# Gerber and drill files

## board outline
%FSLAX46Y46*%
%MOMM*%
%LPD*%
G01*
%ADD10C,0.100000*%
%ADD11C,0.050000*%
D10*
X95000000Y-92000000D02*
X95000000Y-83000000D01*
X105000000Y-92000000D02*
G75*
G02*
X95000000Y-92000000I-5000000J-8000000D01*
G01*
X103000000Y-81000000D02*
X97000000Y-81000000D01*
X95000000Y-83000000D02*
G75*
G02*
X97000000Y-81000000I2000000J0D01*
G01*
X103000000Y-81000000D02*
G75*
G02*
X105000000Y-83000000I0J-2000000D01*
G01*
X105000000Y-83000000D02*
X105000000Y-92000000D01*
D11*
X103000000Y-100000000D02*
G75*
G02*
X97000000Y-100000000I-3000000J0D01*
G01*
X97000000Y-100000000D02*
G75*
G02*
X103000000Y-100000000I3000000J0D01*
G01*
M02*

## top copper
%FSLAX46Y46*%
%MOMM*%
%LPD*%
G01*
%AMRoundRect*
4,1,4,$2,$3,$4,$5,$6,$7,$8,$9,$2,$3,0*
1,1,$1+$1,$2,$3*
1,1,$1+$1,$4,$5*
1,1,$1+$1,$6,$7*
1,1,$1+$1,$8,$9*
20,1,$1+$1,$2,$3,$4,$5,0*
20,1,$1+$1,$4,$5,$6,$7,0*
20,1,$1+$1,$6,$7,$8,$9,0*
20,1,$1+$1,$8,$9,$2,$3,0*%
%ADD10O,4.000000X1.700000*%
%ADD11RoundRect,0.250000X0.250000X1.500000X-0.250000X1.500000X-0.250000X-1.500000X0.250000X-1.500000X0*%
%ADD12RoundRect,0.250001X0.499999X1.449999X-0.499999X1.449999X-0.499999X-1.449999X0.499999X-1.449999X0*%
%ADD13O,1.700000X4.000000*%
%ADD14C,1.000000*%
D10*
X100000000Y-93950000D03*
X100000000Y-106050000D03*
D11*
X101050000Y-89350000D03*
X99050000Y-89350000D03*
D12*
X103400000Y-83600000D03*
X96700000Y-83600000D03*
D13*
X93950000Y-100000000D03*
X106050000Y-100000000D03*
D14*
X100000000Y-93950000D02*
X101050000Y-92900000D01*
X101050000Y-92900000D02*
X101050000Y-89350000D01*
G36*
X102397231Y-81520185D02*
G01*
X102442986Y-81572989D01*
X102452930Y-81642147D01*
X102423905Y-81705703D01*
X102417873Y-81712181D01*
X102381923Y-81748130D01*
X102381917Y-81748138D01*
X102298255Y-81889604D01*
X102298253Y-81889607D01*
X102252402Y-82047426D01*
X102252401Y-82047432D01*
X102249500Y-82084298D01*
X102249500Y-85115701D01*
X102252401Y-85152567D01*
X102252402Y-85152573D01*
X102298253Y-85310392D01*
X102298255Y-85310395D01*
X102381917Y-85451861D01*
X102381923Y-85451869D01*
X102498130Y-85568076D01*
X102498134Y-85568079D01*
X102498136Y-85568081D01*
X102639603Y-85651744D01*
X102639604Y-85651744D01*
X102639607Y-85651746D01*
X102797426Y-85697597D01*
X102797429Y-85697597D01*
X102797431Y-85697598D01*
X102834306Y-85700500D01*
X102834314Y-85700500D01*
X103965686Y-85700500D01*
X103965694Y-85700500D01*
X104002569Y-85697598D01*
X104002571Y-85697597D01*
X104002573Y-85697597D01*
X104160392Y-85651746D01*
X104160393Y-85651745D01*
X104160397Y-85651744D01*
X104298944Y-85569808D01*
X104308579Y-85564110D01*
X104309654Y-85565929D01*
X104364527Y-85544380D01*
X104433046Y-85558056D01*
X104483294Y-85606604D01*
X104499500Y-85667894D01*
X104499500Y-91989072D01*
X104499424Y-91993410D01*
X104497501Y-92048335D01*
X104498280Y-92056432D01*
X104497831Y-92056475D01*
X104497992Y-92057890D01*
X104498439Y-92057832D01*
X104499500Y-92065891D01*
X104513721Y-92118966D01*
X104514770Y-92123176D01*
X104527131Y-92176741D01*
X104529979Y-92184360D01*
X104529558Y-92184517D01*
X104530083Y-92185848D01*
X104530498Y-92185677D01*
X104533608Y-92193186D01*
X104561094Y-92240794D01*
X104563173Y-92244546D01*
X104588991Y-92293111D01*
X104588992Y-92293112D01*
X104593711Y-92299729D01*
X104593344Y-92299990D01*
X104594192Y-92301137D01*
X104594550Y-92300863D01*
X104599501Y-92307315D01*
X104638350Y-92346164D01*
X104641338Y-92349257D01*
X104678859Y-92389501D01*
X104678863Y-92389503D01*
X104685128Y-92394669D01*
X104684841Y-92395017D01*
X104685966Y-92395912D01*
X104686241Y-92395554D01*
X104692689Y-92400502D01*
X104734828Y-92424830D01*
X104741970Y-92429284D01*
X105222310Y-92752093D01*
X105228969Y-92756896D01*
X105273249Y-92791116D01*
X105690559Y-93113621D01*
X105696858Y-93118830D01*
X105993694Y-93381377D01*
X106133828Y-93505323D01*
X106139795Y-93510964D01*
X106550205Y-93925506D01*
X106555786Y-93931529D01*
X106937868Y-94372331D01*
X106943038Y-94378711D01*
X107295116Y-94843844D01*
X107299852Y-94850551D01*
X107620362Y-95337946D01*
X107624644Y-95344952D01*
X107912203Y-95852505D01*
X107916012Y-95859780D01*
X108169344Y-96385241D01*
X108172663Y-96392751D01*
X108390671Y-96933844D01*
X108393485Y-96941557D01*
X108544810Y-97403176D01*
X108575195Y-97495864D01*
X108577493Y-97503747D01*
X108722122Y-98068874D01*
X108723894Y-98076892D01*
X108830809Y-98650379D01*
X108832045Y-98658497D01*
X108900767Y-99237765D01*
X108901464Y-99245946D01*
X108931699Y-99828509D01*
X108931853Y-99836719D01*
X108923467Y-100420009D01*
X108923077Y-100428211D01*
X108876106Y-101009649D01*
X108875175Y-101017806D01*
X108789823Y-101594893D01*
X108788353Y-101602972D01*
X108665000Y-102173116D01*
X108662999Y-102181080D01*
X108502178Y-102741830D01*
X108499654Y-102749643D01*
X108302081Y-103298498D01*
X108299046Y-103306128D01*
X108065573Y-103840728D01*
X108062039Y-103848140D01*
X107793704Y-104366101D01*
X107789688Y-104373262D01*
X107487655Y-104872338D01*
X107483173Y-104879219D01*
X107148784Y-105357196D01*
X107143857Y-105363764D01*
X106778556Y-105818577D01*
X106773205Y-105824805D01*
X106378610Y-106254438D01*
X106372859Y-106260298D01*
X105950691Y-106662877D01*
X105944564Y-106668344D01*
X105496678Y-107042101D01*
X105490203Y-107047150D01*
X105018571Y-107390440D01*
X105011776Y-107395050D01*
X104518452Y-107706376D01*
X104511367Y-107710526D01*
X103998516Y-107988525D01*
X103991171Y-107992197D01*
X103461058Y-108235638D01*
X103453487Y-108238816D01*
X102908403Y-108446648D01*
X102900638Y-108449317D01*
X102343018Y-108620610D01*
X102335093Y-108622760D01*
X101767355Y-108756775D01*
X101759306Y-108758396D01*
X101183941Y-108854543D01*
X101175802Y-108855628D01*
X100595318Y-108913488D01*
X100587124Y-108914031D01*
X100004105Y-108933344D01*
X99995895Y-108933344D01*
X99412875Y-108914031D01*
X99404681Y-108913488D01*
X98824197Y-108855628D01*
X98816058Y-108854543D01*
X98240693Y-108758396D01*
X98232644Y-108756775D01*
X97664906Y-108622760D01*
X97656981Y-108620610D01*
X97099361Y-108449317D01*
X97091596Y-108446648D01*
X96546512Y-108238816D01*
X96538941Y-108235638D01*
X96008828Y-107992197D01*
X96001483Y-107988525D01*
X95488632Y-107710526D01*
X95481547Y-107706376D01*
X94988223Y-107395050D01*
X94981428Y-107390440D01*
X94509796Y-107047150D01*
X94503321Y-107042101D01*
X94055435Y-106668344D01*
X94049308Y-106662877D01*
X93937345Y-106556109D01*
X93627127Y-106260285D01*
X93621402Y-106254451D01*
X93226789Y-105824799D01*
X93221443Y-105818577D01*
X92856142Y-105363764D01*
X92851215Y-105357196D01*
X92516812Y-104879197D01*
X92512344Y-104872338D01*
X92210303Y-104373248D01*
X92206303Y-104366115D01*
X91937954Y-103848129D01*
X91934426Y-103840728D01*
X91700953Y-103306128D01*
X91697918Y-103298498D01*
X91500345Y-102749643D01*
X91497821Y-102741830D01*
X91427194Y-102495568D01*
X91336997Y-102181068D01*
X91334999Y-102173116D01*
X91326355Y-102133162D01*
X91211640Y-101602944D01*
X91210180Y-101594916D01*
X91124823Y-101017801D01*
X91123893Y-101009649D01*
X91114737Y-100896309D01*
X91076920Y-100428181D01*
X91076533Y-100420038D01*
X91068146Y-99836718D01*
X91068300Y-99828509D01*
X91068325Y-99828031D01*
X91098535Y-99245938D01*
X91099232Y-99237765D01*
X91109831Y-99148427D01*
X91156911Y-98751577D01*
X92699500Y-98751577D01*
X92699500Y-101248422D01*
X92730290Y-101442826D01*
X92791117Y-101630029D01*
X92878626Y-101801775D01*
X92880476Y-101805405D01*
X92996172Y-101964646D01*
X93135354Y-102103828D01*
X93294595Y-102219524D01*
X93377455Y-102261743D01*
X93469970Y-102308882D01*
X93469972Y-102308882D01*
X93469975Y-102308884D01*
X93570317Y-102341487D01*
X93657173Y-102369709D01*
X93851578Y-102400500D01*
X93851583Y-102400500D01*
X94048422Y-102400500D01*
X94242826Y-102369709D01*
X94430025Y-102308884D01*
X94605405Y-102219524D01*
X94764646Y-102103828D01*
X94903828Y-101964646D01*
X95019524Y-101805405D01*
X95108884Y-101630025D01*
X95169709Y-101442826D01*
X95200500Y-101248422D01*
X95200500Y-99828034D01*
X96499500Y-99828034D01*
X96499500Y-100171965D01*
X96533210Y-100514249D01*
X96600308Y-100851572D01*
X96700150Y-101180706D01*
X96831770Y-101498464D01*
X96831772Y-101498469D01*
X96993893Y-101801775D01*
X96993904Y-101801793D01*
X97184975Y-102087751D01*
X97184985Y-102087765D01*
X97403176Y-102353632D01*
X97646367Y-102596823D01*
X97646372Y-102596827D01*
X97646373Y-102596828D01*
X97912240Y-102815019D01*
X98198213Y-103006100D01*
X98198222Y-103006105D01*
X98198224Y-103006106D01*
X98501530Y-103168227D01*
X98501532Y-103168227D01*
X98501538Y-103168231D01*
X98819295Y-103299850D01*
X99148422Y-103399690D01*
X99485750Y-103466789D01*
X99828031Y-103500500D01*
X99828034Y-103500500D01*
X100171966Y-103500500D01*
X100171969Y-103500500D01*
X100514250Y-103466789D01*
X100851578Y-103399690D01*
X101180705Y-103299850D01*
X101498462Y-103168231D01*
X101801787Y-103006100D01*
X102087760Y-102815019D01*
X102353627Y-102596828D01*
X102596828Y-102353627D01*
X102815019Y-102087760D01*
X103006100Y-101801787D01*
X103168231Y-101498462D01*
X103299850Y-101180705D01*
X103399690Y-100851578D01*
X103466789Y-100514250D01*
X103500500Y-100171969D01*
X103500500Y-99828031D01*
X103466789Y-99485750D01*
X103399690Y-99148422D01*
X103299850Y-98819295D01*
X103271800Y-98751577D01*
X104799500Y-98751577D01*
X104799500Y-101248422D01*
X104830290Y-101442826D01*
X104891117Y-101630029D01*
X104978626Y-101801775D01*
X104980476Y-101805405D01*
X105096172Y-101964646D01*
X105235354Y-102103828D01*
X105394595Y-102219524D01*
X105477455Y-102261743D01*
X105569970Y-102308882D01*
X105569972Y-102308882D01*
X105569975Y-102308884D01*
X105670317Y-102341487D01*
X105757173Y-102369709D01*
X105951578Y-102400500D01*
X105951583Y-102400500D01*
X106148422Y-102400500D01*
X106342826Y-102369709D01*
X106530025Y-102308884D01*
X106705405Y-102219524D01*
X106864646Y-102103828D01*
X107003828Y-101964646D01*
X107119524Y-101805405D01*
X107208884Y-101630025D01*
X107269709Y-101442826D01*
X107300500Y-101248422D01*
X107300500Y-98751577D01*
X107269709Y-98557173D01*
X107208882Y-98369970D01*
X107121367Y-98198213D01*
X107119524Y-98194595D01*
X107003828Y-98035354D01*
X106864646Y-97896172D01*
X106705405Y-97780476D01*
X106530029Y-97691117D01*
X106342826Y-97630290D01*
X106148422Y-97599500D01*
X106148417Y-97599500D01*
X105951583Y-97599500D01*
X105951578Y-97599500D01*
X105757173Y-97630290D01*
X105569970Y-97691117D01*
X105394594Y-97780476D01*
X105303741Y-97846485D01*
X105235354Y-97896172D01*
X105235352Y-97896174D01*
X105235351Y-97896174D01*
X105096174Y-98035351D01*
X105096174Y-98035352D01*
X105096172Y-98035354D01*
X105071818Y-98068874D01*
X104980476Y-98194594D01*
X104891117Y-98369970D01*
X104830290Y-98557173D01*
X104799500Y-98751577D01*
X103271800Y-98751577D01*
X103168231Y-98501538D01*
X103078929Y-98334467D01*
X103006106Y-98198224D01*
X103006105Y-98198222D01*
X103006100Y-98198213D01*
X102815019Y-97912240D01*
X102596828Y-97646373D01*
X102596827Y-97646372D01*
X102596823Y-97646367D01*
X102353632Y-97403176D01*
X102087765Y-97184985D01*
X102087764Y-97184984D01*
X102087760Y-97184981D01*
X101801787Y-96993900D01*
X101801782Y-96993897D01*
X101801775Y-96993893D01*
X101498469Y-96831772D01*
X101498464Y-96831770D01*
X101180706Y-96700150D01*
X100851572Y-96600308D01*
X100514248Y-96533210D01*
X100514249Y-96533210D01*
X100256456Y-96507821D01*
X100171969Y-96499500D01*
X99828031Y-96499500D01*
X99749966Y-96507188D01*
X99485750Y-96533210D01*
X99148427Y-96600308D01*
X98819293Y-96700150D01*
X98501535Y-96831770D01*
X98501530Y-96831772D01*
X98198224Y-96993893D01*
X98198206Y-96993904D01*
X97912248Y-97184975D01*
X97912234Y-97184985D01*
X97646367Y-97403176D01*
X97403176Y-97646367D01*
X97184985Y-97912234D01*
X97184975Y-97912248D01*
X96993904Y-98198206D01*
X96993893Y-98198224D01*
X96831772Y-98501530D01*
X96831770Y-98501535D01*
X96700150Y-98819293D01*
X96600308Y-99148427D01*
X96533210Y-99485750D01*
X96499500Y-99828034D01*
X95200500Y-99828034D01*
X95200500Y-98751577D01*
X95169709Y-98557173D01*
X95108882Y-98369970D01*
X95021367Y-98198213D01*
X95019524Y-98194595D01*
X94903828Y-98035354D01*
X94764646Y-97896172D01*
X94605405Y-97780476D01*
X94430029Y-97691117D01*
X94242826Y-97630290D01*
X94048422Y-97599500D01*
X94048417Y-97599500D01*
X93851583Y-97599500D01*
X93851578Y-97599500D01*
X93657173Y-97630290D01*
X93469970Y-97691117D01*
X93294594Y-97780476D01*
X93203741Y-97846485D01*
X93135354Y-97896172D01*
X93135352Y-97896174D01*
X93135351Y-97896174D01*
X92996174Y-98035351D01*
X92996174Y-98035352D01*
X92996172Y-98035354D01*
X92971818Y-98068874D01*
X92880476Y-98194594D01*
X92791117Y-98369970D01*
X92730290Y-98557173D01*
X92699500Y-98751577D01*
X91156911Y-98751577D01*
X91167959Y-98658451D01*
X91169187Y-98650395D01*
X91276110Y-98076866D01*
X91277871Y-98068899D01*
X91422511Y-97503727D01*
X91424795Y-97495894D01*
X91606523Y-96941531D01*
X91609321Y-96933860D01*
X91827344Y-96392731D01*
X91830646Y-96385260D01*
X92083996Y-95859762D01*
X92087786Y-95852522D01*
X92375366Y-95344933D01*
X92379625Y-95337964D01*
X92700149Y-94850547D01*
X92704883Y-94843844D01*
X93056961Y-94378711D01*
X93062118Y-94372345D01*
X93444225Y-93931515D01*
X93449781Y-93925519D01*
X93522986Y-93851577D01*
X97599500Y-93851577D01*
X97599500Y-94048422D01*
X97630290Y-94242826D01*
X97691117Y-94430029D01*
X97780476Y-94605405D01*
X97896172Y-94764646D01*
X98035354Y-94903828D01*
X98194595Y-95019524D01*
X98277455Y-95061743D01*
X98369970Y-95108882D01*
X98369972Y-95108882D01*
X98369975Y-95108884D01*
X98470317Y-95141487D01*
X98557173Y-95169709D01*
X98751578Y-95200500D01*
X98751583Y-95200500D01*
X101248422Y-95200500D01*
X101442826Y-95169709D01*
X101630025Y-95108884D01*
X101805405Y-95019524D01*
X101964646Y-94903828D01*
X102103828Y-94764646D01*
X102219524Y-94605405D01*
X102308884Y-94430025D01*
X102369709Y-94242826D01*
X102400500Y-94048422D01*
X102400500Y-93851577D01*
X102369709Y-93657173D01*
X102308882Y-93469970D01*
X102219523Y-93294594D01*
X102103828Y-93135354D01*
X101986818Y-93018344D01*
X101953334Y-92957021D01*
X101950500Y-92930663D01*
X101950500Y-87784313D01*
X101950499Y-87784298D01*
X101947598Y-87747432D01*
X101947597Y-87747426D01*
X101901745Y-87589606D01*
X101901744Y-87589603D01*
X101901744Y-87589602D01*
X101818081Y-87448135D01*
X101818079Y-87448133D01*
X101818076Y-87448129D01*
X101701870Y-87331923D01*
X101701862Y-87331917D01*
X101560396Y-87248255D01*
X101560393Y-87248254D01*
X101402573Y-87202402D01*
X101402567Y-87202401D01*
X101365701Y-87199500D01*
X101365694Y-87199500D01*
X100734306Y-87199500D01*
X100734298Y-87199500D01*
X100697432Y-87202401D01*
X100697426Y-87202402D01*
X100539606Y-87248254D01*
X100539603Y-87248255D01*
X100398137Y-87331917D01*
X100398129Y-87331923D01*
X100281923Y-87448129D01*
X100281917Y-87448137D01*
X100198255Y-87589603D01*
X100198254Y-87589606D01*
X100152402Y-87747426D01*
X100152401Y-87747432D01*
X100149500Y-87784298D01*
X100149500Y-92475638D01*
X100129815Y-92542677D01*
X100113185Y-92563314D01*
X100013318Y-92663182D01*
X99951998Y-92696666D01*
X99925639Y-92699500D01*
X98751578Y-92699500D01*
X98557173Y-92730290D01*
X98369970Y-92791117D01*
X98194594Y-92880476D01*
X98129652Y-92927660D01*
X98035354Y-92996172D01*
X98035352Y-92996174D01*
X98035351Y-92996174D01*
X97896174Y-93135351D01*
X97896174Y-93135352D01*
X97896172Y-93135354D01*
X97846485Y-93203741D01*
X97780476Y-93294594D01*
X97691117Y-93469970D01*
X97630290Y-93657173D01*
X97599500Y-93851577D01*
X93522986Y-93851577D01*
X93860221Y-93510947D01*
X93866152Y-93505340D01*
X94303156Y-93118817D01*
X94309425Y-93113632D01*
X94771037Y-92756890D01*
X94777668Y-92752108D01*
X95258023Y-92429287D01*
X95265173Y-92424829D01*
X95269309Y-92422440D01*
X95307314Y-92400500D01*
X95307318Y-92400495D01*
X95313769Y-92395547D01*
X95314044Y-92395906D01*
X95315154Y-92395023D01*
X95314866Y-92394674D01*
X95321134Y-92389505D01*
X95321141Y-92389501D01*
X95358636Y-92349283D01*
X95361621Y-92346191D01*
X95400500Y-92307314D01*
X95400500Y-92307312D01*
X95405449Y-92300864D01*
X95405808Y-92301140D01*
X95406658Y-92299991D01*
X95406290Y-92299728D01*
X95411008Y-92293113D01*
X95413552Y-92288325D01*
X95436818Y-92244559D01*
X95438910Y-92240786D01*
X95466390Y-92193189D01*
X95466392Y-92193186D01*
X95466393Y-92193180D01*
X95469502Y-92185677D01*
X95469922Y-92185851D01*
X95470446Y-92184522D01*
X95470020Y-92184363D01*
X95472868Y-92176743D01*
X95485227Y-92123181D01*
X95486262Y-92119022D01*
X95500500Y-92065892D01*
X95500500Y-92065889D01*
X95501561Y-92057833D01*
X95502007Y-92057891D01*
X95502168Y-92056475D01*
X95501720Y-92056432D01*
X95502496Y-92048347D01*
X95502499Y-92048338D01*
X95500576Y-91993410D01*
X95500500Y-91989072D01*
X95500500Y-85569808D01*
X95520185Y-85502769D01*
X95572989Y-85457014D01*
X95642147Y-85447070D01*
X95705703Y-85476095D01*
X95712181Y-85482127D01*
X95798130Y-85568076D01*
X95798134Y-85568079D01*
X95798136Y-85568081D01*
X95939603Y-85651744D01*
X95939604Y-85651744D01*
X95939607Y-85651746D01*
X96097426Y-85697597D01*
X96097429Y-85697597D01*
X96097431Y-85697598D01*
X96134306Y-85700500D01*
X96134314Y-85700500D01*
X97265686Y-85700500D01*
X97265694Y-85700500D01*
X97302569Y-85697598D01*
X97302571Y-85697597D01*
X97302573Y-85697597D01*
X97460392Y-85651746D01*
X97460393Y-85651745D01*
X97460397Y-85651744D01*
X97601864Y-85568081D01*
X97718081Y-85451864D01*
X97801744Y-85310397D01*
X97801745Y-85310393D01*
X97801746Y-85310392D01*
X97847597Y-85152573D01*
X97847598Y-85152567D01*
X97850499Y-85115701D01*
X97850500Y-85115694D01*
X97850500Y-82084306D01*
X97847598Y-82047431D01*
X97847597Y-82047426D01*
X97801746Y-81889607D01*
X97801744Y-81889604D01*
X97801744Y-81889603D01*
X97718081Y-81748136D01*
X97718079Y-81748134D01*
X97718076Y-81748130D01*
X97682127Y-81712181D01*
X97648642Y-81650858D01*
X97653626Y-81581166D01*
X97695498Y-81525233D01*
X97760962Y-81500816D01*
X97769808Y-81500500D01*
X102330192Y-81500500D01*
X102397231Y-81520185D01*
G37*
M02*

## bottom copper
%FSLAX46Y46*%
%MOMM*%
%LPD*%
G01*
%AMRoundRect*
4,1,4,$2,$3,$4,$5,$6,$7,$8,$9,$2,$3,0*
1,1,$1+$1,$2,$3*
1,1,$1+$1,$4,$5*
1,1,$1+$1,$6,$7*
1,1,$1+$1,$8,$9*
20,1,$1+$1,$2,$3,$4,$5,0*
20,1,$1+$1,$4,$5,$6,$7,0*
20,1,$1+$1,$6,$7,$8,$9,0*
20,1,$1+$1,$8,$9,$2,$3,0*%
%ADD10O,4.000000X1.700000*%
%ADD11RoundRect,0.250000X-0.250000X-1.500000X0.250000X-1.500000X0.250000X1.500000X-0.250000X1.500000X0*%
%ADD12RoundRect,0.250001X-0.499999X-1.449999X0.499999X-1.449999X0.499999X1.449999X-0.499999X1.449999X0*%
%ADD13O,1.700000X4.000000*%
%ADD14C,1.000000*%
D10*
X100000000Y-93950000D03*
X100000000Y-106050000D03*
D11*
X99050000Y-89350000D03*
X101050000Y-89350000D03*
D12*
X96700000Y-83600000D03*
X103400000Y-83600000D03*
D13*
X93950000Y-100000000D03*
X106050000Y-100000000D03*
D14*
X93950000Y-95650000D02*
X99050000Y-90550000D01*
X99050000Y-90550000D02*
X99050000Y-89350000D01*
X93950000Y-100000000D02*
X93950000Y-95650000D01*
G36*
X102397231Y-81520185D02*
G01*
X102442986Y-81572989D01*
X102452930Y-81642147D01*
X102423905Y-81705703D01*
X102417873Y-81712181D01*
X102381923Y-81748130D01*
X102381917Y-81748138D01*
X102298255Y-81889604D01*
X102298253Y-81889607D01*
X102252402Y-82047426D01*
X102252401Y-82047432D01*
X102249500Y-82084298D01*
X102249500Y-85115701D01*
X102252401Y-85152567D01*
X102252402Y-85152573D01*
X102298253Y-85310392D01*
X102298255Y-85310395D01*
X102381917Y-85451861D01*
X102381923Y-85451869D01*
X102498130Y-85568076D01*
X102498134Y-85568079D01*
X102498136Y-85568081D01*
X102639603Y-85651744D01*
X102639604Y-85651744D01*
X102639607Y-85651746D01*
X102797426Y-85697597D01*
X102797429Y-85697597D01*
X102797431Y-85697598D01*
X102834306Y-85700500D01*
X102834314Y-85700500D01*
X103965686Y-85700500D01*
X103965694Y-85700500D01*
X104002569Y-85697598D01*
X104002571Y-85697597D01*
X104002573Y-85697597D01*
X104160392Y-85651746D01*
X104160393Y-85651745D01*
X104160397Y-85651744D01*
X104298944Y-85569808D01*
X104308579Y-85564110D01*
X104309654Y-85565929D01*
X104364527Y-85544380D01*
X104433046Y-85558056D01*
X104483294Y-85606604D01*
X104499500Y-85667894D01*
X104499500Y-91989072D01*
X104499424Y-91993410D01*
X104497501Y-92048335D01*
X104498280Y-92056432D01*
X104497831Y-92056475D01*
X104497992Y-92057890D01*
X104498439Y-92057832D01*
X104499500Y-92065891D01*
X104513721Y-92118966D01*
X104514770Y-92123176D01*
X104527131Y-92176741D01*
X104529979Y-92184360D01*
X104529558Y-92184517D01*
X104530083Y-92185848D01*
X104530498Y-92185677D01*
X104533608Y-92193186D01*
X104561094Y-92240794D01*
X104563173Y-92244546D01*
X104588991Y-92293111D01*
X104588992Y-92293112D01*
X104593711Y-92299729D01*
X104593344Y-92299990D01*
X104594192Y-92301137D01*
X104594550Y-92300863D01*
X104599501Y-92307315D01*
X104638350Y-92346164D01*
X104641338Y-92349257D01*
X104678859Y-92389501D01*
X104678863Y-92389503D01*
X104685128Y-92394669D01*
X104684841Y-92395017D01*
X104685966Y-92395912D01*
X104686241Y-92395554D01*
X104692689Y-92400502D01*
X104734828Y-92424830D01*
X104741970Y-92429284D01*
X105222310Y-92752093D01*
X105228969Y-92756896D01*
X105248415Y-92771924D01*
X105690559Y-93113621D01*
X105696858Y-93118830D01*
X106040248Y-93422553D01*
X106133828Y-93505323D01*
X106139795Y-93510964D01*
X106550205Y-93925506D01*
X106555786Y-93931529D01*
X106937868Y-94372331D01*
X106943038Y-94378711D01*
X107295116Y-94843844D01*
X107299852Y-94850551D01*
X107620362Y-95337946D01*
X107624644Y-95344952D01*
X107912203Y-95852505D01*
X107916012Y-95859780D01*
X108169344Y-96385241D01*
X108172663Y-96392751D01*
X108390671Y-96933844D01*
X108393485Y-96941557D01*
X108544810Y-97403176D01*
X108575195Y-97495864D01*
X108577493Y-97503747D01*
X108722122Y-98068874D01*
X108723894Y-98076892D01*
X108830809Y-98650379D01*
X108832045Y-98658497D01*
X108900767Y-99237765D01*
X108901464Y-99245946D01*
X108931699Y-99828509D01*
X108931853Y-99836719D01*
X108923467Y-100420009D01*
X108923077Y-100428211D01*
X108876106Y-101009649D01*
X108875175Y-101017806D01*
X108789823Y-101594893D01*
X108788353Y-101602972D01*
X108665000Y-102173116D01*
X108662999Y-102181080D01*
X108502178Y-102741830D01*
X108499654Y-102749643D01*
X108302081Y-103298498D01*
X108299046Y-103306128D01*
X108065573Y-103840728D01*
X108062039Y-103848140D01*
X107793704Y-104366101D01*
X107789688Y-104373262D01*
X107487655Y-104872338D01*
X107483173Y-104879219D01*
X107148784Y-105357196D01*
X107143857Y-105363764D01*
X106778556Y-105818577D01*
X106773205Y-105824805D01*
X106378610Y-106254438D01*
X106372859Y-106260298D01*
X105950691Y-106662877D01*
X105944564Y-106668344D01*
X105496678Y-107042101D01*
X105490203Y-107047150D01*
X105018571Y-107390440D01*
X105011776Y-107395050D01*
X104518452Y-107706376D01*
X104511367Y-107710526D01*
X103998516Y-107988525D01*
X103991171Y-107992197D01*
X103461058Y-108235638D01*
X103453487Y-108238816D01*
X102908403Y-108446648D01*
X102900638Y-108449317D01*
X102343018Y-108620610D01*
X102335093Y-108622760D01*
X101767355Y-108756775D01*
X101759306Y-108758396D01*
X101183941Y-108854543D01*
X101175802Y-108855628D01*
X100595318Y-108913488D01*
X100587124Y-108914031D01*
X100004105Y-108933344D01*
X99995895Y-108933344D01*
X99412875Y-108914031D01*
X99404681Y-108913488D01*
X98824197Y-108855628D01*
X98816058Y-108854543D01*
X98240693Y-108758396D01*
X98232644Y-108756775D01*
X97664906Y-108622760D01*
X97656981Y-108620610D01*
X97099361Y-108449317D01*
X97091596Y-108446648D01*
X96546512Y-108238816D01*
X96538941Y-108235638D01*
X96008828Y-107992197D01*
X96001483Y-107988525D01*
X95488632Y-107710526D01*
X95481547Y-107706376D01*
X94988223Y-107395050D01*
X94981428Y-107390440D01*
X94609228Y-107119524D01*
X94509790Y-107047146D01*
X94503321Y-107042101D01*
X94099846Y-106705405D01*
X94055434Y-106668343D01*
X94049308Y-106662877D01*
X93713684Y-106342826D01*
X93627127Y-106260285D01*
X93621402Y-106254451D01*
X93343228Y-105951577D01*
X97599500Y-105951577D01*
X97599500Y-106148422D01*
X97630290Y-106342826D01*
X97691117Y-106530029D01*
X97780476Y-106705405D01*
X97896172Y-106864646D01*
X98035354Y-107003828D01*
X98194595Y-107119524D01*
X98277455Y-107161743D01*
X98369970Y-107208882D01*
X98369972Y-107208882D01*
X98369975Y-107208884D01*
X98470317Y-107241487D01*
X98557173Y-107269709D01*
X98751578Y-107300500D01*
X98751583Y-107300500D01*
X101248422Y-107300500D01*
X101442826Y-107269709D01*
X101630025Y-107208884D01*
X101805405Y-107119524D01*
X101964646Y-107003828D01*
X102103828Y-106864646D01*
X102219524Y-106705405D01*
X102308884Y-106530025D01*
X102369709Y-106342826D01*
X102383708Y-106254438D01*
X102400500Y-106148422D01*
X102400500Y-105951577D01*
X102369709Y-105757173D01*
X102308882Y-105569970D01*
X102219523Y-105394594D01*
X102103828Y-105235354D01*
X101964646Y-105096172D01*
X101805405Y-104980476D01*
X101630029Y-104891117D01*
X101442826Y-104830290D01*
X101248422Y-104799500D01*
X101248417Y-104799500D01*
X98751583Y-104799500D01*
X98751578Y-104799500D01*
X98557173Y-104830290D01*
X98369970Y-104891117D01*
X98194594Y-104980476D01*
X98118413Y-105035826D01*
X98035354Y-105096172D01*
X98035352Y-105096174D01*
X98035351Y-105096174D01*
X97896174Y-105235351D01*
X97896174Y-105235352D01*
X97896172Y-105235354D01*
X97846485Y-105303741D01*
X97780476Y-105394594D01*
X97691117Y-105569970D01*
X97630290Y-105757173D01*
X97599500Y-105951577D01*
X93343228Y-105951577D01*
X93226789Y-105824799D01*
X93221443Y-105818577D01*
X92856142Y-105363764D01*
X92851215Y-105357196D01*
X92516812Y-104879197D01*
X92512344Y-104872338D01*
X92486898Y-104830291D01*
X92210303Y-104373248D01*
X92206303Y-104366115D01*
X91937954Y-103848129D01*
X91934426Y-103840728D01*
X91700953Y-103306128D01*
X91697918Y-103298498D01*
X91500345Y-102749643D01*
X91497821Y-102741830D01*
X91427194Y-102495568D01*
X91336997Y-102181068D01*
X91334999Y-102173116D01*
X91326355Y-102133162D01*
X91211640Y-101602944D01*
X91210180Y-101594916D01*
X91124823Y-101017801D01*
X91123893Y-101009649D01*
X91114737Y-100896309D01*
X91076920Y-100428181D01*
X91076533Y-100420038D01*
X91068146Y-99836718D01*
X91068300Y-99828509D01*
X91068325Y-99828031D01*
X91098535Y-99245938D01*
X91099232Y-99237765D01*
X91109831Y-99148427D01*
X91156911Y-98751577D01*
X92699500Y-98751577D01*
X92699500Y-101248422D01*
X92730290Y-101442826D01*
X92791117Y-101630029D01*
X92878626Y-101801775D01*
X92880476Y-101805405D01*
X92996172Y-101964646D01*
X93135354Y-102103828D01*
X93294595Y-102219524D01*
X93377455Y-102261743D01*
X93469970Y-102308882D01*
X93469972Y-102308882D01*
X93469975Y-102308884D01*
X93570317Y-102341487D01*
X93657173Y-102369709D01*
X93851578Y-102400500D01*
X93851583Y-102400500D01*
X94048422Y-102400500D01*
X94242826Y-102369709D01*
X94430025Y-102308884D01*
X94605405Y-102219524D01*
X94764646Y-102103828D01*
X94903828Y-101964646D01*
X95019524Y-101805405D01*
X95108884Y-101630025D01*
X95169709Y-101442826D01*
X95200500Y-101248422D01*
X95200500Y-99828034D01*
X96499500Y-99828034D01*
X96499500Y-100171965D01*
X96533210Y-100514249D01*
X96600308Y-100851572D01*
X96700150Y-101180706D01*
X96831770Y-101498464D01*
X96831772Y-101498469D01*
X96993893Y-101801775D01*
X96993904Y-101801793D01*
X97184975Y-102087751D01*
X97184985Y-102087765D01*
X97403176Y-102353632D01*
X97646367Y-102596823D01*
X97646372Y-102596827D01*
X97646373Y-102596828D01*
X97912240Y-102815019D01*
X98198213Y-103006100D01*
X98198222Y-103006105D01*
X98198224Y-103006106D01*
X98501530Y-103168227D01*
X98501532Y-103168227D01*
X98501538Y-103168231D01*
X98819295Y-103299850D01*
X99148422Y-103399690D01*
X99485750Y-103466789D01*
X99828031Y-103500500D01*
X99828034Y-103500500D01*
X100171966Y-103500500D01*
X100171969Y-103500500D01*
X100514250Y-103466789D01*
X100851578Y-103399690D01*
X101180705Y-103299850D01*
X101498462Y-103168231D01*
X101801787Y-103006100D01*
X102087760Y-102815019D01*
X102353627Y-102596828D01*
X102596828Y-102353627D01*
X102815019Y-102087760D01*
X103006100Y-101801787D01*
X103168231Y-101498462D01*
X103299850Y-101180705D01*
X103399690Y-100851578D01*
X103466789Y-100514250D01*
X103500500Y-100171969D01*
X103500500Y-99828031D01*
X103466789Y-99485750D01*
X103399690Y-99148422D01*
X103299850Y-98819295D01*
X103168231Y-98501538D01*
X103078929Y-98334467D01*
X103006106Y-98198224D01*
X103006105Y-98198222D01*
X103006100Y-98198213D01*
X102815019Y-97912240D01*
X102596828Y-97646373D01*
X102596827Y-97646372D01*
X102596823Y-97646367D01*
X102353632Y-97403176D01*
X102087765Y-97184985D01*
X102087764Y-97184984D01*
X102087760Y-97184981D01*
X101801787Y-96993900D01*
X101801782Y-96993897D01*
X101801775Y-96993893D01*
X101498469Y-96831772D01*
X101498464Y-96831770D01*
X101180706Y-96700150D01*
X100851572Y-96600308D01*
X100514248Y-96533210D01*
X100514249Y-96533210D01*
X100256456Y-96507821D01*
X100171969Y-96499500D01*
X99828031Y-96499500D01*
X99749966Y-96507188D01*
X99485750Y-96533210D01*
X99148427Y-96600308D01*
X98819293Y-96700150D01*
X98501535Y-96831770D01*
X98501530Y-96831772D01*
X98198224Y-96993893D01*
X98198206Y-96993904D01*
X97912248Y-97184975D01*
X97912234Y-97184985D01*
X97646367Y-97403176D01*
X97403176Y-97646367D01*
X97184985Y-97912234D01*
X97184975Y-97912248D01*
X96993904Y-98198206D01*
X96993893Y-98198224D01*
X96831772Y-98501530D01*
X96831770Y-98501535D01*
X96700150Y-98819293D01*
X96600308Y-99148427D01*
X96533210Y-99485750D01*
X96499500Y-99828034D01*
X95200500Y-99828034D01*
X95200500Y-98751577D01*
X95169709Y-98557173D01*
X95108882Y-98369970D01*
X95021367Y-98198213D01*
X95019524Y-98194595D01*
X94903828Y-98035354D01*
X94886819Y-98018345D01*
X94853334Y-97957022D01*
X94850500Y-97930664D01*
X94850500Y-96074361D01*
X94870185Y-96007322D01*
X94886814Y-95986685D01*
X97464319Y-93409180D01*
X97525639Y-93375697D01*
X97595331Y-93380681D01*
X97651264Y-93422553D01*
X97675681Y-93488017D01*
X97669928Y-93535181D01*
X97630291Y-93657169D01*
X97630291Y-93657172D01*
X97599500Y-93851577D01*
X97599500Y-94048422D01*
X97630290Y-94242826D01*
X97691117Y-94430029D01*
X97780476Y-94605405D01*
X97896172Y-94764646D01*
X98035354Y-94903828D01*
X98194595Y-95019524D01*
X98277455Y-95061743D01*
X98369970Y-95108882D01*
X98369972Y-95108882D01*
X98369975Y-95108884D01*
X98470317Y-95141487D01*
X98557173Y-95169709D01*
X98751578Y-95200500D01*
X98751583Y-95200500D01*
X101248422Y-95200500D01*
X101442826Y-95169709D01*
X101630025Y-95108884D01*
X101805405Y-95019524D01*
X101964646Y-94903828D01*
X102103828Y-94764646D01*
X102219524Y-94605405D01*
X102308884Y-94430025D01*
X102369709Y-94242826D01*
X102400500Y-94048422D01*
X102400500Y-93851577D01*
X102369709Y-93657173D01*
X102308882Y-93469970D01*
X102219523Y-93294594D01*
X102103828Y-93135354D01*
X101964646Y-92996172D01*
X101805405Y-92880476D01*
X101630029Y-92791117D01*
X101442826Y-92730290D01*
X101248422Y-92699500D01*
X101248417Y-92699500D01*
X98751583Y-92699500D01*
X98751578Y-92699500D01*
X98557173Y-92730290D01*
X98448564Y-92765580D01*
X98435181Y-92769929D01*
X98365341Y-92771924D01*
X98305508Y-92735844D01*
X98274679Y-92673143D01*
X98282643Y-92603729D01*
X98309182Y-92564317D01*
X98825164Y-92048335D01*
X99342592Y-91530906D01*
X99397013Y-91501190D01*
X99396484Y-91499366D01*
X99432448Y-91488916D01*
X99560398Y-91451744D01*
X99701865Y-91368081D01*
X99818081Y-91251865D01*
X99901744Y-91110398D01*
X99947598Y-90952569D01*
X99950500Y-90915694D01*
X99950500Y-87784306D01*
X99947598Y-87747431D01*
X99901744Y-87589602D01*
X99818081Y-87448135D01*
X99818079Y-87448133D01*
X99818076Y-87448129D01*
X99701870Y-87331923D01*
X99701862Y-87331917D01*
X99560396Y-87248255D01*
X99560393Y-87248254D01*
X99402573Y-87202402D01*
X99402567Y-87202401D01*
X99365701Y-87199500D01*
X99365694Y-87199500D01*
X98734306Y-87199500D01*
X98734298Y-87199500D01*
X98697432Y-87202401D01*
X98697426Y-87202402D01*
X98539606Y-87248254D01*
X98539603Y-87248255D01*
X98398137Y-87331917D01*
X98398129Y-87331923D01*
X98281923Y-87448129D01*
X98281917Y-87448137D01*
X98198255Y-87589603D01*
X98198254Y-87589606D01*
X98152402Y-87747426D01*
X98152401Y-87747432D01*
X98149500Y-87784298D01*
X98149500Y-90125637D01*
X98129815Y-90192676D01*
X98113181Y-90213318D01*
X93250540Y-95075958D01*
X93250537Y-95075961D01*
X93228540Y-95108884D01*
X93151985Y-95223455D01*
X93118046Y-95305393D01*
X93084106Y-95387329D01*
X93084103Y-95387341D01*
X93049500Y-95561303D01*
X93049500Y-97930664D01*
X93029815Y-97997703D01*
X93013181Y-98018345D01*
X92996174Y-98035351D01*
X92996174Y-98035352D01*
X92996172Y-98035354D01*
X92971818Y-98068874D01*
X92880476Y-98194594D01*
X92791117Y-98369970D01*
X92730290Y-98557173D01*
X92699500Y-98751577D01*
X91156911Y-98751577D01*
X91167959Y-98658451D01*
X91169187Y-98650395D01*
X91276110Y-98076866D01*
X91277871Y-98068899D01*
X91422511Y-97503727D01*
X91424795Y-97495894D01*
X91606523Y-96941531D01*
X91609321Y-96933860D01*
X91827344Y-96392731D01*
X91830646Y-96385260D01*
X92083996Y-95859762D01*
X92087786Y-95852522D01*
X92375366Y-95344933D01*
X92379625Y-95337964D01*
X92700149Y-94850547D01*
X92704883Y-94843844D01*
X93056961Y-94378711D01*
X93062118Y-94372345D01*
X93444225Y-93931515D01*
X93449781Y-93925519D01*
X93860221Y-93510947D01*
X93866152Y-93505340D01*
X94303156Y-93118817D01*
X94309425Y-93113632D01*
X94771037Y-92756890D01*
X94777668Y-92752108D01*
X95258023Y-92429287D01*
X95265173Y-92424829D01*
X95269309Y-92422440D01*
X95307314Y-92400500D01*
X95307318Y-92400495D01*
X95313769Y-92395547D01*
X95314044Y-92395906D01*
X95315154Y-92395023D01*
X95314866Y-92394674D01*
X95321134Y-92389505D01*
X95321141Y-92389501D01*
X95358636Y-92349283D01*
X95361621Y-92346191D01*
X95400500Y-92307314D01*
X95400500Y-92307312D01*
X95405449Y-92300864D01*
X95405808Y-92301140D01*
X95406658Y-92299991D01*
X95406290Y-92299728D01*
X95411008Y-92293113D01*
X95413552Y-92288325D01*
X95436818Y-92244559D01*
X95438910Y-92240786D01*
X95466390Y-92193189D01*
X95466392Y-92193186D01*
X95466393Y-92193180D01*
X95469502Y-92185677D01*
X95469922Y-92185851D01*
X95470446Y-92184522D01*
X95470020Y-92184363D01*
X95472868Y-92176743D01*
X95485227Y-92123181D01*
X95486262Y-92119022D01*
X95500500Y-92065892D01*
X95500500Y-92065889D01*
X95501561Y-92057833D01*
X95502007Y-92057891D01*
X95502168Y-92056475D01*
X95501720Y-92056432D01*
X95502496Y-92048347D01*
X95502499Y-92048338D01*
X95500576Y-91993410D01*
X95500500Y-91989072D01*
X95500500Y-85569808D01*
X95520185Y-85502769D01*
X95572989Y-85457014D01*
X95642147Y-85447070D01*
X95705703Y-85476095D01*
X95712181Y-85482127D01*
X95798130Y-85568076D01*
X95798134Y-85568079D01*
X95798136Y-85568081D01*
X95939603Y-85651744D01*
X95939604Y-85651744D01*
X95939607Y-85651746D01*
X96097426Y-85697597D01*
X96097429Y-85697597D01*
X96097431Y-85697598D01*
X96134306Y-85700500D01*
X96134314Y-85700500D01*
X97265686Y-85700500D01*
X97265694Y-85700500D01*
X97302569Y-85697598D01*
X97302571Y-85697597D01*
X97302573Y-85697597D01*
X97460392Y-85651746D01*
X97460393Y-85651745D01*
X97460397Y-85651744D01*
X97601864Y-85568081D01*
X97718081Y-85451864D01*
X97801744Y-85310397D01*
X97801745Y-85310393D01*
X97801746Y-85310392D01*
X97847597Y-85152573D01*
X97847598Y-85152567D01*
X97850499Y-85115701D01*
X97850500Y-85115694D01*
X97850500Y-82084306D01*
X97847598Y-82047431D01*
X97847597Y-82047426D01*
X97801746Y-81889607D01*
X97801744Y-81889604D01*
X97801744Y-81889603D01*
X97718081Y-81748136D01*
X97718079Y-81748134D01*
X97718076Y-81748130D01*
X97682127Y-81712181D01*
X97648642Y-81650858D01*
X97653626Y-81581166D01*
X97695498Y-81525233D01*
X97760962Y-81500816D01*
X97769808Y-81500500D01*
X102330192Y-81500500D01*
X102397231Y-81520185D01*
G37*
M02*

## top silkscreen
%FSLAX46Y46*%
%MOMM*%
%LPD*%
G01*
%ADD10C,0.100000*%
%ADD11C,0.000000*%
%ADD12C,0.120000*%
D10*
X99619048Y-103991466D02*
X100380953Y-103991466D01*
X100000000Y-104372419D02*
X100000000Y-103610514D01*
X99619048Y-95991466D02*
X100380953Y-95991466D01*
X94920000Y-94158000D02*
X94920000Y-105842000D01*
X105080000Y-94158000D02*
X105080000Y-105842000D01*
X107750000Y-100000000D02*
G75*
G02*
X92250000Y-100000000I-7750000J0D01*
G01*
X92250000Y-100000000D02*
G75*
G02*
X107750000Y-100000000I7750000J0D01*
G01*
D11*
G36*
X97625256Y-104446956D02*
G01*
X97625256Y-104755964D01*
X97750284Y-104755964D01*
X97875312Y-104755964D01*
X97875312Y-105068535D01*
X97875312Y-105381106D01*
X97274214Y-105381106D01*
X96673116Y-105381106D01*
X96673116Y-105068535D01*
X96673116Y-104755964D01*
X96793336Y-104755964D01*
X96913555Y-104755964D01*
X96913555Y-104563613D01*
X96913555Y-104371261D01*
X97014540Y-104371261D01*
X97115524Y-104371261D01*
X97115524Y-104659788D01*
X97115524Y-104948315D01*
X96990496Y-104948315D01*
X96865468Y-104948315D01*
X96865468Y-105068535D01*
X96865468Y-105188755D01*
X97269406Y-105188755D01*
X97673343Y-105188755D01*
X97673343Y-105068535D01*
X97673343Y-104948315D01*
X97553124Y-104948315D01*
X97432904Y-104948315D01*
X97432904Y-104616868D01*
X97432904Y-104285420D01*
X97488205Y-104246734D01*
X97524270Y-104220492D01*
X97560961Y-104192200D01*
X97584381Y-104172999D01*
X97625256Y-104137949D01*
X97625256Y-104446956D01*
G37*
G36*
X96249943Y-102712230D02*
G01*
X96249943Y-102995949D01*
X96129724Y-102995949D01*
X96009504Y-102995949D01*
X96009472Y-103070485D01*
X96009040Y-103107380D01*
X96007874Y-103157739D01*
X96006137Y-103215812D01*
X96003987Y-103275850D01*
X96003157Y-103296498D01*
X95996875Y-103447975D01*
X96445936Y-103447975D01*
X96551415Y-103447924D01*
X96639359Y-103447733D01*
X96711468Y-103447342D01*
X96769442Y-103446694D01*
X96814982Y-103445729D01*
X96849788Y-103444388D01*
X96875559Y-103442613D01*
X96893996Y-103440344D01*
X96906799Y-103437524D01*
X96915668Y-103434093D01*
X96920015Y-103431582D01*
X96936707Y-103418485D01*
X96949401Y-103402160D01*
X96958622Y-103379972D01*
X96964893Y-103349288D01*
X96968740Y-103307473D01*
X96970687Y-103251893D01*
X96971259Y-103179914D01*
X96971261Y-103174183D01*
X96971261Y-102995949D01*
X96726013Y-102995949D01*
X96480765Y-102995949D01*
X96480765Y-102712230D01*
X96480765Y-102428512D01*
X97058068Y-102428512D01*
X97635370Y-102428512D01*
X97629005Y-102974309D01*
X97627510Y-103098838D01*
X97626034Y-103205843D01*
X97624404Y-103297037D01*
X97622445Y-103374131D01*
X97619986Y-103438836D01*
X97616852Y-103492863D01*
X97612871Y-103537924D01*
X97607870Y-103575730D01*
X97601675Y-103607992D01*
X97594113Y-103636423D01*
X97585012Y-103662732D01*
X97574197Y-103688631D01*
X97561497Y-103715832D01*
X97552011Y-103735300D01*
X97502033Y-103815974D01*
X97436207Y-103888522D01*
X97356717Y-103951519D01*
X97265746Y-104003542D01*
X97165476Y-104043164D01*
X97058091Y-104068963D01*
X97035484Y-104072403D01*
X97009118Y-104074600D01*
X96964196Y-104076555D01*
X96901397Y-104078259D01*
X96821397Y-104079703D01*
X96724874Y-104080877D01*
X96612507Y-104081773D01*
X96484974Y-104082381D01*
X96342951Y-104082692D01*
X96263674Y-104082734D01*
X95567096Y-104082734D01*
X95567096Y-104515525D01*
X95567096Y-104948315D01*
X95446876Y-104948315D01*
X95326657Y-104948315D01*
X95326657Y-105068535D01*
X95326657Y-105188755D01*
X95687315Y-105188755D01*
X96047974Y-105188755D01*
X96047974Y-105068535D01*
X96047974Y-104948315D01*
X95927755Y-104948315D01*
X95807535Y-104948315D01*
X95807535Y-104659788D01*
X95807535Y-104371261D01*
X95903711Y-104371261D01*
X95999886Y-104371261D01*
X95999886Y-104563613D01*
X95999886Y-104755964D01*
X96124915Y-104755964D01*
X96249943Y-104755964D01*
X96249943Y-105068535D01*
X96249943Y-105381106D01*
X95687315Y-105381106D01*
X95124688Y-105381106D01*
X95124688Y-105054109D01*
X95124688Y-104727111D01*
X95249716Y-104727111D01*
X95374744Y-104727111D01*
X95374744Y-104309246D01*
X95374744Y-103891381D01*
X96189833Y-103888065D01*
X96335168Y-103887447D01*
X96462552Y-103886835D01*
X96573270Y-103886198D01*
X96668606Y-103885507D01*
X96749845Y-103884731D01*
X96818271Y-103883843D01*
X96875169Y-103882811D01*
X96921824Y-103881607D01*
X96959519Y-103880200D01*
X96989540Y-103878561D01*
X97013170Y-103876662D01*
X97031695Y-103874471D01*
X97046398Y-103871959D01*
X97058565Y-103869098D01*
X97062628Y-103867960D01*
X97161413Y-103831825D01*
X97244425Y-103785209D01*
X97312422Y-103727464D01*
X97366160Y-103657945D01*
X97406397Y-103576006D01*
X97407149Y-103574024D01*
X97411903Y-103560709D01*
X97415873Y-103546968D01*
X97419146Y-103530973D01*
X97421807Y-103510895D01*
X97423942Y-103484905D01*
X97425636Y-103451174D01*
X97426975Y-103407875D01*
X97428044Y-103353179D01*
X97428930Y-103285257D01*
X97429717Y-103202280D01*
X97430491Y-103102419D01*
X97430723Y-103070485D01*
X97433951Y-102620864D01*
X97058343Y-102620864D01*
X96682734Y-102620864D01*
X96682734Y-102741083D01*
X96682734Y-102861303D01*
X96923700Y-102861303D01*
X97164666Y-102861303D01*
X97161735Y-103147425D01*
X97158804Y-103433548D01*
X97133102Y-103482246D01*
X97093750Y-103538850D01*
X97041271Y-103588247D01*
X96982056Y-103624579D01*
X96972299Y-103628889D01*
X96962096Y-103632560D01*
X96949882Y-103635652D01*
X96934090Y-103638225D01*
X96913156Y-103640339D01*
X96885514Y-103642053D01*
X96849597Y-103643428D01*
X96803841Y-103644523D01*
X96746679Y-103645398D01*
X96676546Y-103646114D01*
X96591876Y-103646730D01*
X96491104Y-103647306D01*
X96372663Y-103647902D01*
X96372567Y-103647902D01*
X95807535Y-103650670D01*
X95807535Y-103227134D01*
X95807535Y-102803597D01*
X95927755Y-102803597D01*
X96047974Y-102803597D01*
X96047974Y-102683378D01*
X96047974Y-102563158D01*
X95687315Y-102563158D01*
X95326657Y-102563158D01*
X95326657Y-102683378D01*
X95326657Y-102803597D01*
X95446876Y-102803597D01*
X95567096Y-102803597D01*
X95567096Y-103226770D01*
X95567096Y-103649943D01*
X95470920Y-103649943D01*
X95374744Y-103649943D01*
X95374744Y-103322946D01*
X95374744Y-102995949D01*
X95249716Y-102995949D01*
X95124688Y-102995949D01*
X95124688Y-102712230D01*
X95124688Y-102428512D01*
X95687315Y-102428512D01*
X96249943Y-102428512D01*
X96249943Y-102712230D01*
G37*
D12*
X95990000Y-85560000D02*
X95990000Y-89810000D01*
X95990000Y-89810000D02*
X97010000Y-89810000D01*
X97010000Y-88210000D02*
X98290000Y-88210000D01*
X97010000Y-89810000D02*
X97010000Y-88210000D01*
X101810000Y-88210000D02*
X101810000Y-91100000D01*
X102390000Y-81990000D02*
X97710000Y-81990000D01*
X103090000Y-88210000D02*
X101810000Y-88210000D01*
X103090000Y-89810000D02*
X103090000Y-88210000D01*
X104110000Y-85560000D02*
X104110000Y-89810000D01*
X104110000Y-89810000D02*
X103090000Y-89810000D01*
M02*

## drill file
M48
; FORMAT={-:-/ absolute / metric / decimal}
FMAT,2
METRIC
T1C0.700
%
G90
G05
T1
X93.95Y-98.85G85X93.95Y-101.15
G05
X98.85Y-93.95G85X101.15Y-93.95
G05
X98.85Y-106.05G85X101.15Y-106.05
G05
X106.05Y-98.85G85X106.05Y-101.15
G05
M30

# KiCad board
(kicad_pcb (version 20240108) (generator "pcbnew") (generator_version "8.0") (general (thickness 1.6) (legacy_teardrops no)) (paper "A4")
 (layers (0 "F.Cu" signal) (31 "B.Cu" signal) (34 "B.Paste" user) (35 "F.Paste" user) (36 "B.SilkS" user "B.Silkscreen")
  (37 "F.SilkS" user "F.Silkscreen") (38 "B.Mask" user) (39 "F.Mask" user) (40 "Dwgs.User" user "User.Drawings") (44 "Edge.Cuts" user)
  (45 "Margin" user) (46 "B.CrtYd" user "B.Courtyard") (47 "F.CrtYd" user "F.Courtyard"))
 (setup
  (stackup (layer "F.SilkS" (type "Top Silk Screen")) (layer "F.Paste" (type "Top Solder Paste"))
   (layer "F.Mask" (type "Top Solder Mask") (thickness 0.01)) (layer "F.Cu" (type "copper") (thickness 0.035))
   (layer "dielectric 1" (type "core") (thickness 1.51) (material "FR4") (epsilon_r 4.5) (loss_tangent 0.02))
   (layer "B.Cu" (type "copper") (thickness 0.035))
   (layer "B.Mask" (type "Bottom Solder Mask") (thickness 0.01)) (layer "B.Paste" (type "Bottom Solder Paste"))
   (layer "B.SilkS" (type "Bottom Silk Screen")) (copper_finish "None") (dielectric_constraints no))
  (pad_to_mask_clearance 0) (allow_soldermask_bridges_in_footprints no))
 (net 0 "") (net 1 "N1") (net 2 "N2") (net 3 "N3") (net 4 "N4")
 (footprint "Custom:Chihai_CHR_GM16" (layer "F.Cu") (at 100 100)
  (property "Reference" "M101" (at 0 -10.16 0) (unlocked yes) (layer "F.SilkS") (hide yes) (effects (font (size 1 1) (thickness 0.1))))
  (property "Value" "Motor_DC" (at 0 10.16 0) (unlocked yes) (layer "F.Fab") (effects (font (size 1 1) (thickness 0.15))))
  (fp_line (start -5.08 -5.842) (end -5.08 5.842) (stroke (width 0.1) (type default)) (layer "F.SilkS"))
  (fp_line (start 5.08 -5.842) (end 5.08 5.842) (stroke (width 0.1) (type default)) (layer "F.SilkS"))
  (fp_circle (center 0 0) (end 7.75 0) (stroke (width 0.1) (type default)) (fill none) (layer "F.SilkS"))
  (fp_circle (center 0 0) (end 3 0) (stroke (width 0.05) (type default)) (fill none) (layer "Edge.Cuts"))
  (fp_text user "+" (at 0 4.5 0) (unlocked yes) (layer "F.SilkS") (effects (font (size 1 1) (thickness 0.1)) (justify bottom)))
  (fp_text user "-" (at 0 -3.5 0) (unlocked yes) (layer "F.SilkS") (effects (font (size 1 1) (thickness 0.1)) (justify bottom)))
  (pad "1" thru_hole oval (at 0 -6.05) (size 4 1.7) (drill oval 3 0.7) (layers "*.Cu" "*.Mask") (remove_unused_layers no) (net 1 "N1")
   (thermal_bridge_angle 45))
  (pad "2" thru_hole oval (at 0 6.05) (size 4 1.7) (drill oval 3 0.7) (layers "*.Cu" "*.Mask") (remove_unused_layers no) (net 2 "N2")
   (thermal_bridge_angle 45)))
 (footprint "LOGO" (layer "F.Cu") (at 96.5 103.9)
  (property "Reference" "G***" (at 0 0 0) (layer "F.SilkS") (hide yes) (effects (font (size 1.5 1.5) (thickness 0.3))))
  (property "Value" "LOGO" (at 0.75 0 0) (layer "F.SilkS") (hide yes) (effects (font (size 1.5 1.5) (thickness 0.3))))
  (fp_poly
   (pts (xy 1.125256 0.546956) (xy 1.125256 0.855964) (xy 1.250284 0.855964) (xy 1.375312 0.855964) (xy 1.375312 1.168535)
    (xy 1.375312 1.481106) (xy 0.774214 1.481106) (xy 0.173116 1.481106) (xy 0.173116 1.168535) (xy 0.173116 0.855964)
    (xy 0.293336 0.855964) (xy 0.413555 0.855964) (xy 0.413555 0.663613) (xy 0.413555 0.471261) (xy 0.51454 0.471261) (xy 0.615524 0.471261)
    (xy 0.615524 0.759788) (xy 0.615524 1.048315) (xy 0.490496 1.048315) (xy 0.365468 1.048315) (xy 0.365468 1.168535)
    (xy 0.365468 1.288755) (xy 0.769406 1.288755) (xy 1.173343 1.288755) (xy 1.173343 1.168535) (xy 1.173343 1.048315)
    (xy 1.053124 1.048315) (xy 0.932904 1.048315) (xy 0.932904 0.716868) (xy 0.932904 0.38542) (xy 0.988205 0.346734) (xy 1.02427 0.320492)
    (xy 1.060961 0.2922) (xy 1.084381 0.272999) (xy 1.125256 0.237949))
   (stroke (width 0) (type solid)) (fill solid) (layer "F.SilkS"))
  (fp_poly
   (pts (xy -0.250057 -1.18777) (xy -0.250057 -0.904051) (xy -0.370276 -0.904051) (xy -0.490496 -0.904051) (xy -0.490528 -0.829515)
    (xy -0.49096 -0.79262) (xy -0.492126 -0.742261) (xy -0.493863 -0.684188) (xy -0.496013 -0.62415) (xy -0.496843 -0.603502)
    (xy -0.503125 -0.452025) (xy -0.054064 -0.452025) (xy 0.051415 -0.452076) (xy 0.139359 -0.452267) (xy 0.211468 -0.452658)
    (xy 0.269442 -0.453306) (xy 0.314982 -0.454271) (xy 0.349788 -0.455612) (xy 0.375559 -0.457387) (xy 0.393996 -0.459656)
    (xy 0.406799 -0.462476) (xy 0.415668 -0.465907) (xy 0.420015 -0.468418) (xy 0.436707 -0.481515) (xy 0.449401 -0.49784)
    (xy 0.458622 -0.520028) (xy 0.464893 -0.550712) (xy 0.46874 -0.592527) (xy 0.470687 -0.648107) (xy 0.471259 -0.720086)
    (xy 0.471261 -0.725817) (xy 0.471261 -0.904051) (xy 0.226013 -0.904051) (xy -0.019235 -0.904051) (xy -0.019235 -1.18777)
    (xy -0.019235 -1.471488) (xy 0.558068 -1.471488) (xy 1.13537 -1.471488) (xy 1.129005 -0.925691) (xy 1.12751 -0.801162)
    (xy 1.126034 -0.694157) (xy 1.124404 -0.602963) (xy 1.122445 -0.525869) (xy 1.119986 -0.461164) (xy 1.116852 -0.407137)
    (xy 1.112871 -0.362076) (xy 1.10787 -0.32427) (xy 1.101675 -0.292008) (xy 1.094113 -0.263577) (xy 1.085012 -0.237268)
    (xy 1.074197 -0.211369) (xy 1.061497 -0.184168) (xy 1.052011 -0.1647) (xy 1.002033 -0.084026) (xy 0.936207 -0.011478)
    (xy 0.856717 0.051519) (xy 0.765746 0.103542) (xy 0.665476 0.143164) (xy 0.558091 0.168963) (xy 0.535484 0.172403) (xy 0.509118 0.1746)
    (xy 0.464196 0.176555) (xy 0.401397 0.178259) (xy 0.321397 0.179703) (xy 0.224874 0.180877) (xy 0.112507 0.181773)
    (xy -0.015026 0.182381) (xy -0.157049 0.182692) (xy -0.236326 0.182734) (xy -0.932904 0.182734) (xy -0.932904 0.615525)
    (xy -0.932904 1.048315) (xy -1.053124 1.048315) (xy -1.173343 1.048315) (xy -1.173343 1.168535) (xy -1.173343 1.288755)
    (xy -0.812685 1.288755) (xy -0.452026 1.288755) (xy -0.452026 1.168535) (xy -0.452026 1.048315) (xy -0.572245 1.048315)
    (xy -0.692465 1.048315) (xy -0.692465 0.759788) (xy -0.692465 0.471261) (xy -0.596289 0.471261) (xy -0.500114 0.471261)
    (xy -0.500114 0.663613) (xy -0.500114 0.855964) (xy -0.375085 0.855964) (xy -0.250057 0.855964) (xy -0.250057 1.168535)
    (xy -0.250057 1.481106) (xy -0.812685 1.481106) (xy -1.375312 1.481106) (xy -1.375312 1.154109) (xy -1.375312 0.827111)
    (xy -1.250284 0.827111) (xy -1.125256 0.827111) (xy -1.125256 0.409246) (xy -1.125256 -0.008619) (xy -0.310167 -0.011935)
    (xy -0.164832 -0.012553) (xy -0.037448 -0.013165) (xy 0.07327 -0.013802) (xy 0.168606 -0.014493) (xy 0.249845 -0.015269)
    (xy 0.318271 -0.016157) (xy 0.375169 -0.017189) (xy 0.421824 -0.018393) (xy 0.459519 -0.0198) (xy 0.48954 -0.021439)
    (xy 0.51317 -0.023338) (xy 0.531695 -0.025529) (xy 0.546398 -0.028041) (xy 0.558565 -0.030902) (xy 0.562628 -0.03204)
    (xy 0.661413 -0.068175) (xy 0.744425 -0.114791) (xy 0.812422 -0.172536) (xy 0.86616 -0.242055) (xy 0.906397 -0.323994)
    (xy 0.907149 -0.325976) (xy 0.911903 -0.339291) (xy 0.915873 -0.353032) (xy 0.919146 -0.369027) (xy 0.921807 -0.389105)
    (xy 0.923942 -0.415095) (xy 0.925636 -0.448826) (xy 0.926975 -0.492125) (xy 0.928044 -0.546821) (xy 0.92893 -0.614743)
    (xy 0.929717 -0.69772) (xy 0.930491 -0.797581) (xy 0.930723 -0.829515) (xy 0.933951 -1.279136) (xy 0.558343 -1.279136)
    (xy 0.182734 -1.279136) (xy 0.182734 -1.158917) (xy 0.182734 -1.038697) (xy 0.4237 -1.038697) (xy 0.664666 -1.038697)
    (xy 0.661735 -0.752575) (xy 0.658804 -0.466452) (xy 0.633102 -0.417754) (xy 0.59375 -0.36115) (xy 0.541271 -0.311753)
    (xy 0.482056 -0.275421) (xy 0.472299 -0.271111) (xy 0.462096 -0.26744) (xy 0.449882 -0.264348) (xy 0.43409 -0.261775)
    (xy 0.413156 -0.259661) (xy 0.385514 -0.257947) (xy 0.349597 -0.256572) (xy 0.303841 -0.255477) (xy 0.246679 -0.254602)
    (xy 0.176546 -0.253886) (xy 0.091876 -0.25327) (xy -0.008896 -0.252694) (xy -0.127337 -0.252098) (xy -0.127433 -0.252098)
    (xy -0.692465 -0.24933) (xy -0.692465 -0.672866) (xy -0.692465 -1.096403) (xy -0.572245 -1.096403) (xy -0.452026 -1.096403)
    (xy -0.452026 -1.216622) (xy -0.452026 -1.336842) (xy -0.812685 -1.336842) (xy -1.173343 -1.336842) (xy -1.173343 -1.216622)
    (xy -1.173343 -1.096403) (xy -1.053124 -1.096403) (xy -0.932904 -1.096403) (xy -0.932904 -0.67323) (xy -0.932904 -0.250057)
    (xy -1.02908 -0.250057) (xy -1.125256 -0.250057) (xy -1.125256 -0.577054) (xy -1.125256 -0.904051) (xy -1.250284 -0.904051)
    (xy -1.375312 -0.904051) (xy -1.375312 -1.18777) (xy -1.375312 -1.471488) (xy -0.812685 -1.471488) (xy -0.250057 -1.471488))
   (stroke (width 0) (type solid)) (fill solid) (layer "F.SilkS")))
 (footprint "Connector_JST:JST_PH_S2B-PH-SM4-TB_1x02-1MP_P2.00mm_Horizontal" (layer "F.Cu") (at 100.05 86.5 180)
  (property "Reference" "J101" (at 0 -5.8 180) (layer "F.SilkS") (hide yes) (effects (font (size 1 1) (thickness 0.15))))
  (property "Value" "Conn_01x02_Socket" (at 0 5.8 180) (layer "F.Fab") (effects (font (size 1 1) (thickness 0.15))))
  (fp_line (start 4.06 0.94) (end 4.06 -3.31) (stroke (width 0.12) (type solid)) (layer "F.SilkS"))
  (fp_line (start 4.06 -3.31) (end 3.04 -3.31) (stroke (width 0.12) (type solid)) (layer "F.SilkS"))
  (fp_line (start 3.04 -1.71) (end 1.76 -1.71) (stroke (width 0.12) (type solid)) (layer "F.SilkS"))
  (fp_line (start 3.04 -3.31) (end 3.04 -1.71) (stroke (width 0.12) (type solid)) (layer "F.SilkS"))
  (fp_line (start -1.76 -1.71) (end -1.76 -4.6) (stroke (width 0.12) (type solid)) (layer "F.SilkS"))
  (fp_line (start -2.34 4.51) (end 2.34 4.51) (stroke (width 0.12) (type solid)) (layer "F.SilkS"))
  (fp_line (start -3.04 -1.71) (end -1.76 -1.71) (stroke (width 0.12) (type solid)) (layer "F.SilkS"))
  (fp_line (start -3.04 -3.31) (end -3.04 -1.71) (stroke (width 0.12) (type solid)) (layer "F.SilkS"))
  (fp_line (start -4.06 0.94) (end -4.06 -3.31) (stroke (width 0.12) (type solid)) (layer "F.SilkS"))
  (fp_line (start -4.06 -3.31) (end -3.04 -3.31) (stroke (width 0.12) (type solid)) (layer "F.SilkS"))
  (pad "1" smd roundrect (at -1 -2.85 180) (size 1 3.5) (layers "F.Cu" "F.Paste" "F.Mask") (roundrect_rratio 0.25) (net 1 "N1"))
  (pad "2" smd roundrect (at 1 -2.85 180) (size 1 3.5) (layers "F.Cu" "F.Paste" "F.Mask") (roundrect_rratio 0.25) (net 2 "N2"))
  (pad "MP" smd roundrect (at -3.35 2.9 180) (size 1.5 3.4) (layers "F.Cu" "F.Paste" "F.Mask") (roundrect_rratio 0.166667))
  (pad "MP" smd roundrect (at 3.35 2.9 180) (size 1.5 3.4) (layers "F.Cu" "F.Paste" "F.Mask") (roundrect_rratio 0.166667)))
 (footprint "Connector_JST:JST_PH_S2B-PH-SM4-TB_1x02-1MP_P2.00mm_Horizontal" (layer "B.Cu") (at 100.05 86.5)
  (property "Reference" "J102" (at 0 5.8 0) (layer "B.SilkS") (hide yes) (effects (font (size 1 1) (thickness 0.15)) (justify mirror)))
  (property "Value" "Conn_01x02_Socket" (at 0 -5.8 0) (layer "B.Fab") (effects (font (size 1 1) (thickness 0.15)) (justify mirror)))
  (pad "1" smd roundrect (at -1 2.85) (size 1 3.5) (layers "B.Cu" "B.Paste" "B.Mask") (roundrect_rratio 0.25) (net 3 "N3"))
  (pad "2" smd roundrect (at 1 2.85) (size 1 3.5) (layers "B.Cu" "B.Paste" "B.Mask") (roundrect_rratio 0.25) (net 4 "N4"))
  (pad "MP" smd roundrect (at -3.35 -2.9) (size 1.5 3.4) (layers "B.Cu" "B.Paste" "B.Mask") (roundrect_rratio 0.166667))
  (pad "MP" smd roundrect (at 3.35 -2.9) (size 1.5 3.4) (layers "B.Cu" "B.Paste" "B.Mask") (roundrect_rratio 0.166667)))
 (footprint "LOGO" (layer "B.Cu") (at 104 103.4 180)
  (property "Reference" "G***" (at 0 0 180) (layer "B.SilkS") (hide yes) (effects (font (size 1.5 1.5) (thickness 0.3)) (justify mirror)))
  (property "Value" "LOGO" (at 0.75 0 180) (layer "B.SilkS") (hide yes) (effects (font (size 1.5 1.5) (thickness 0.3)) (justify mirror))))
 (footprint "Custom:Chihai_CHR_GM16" (layer "B.Cu") (at 100 100 -90)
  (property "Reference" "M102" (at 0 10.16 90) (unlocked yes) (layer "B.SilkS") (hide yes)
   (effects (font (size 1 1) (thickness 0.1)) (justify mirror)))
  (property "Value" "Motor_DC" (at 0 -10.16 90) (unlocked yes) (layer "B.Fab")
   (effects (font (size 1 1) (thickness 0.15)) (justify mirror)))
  (pad "1" thru_hole oval (at 0 6.05 270) (size 4 1.7) (drill oval 3 0.7) (layers "*.Cu" "*.Mask") (remove_unused_layers no) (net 3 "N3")
   (thermal_bridge_angle 45))
  (pad "2" thru_hole oval (at 0 -6.05 270) (size 4 1.7) (drill oval 3 0.7) (layers "*.Cu" "*.Mask") (remove_unused_layers no) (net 4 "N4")
   (thermal_bridge_angle 45)))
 (gr_line (start 95 92) (end 95 83) (stroke (width 0.1) (type default)) (layer "Edge.Cuts"))
 (gr_arc (start 105 92) (mid 100 109.433981) (end 95 92) (stroke (width 0.1) (type default)) (layer "Edge.Cuts"))
 (gr_line (start 103 81) (end 97 81) (stroke (width 0.1) (type default)) (layer "Edge.Cuts"))
 (gr_arc (start 95 83) (mid 95.585786 81.585786) (end 97 81) (stroke (width 0.1) (type default)) (layer "Edge.Cuts"))
 (gr_arc (start 103 81) (mid 104.414214 81.585786) (end 105 83) (stroke (width 0.1) (type default)) (layer "Edge.Cuts"))
 (gr_line (start 105 83) (end 105 92) (stroke (width 0.1) (type default)) (layer "Edge.Cuts"))
 (segment (start 100 93.95) (end 101.05 92.9) (width 1) (layer "F.Cu") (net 1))
 (segment (start 101.05 92.9) (end 101.05 89.35) (width 1) (layer "F.Cu") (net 1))
 (segment (start 93.95 95.65) (end 99.05 90.55) (width 1) (layer "B.Cu") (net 3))
 (segment (start 99.05 90.55) (end 99.05 89.35) (width 1) (layer "B.Cu") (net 3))
 (segment (start 93.95 100) (end 93.95 95.65) (width 1) (layer "B.Cu") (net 3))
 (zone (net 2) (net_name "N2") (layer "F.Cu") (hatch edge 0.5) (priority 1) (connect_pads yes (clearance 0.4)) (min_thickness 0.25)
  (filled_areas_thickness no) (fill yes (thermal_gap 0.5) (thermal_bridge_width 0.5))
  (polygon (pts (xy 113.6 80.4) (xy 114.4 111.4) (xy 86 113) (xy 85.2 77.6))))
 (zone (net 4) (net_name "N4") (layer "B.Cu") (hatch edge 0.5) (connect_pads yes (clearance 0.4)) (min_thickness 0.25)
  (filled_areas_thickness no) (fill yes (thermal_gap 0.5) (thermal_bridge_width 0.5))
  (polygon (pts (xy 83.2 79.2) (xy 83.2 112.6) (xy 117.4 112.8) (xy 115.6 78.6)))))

